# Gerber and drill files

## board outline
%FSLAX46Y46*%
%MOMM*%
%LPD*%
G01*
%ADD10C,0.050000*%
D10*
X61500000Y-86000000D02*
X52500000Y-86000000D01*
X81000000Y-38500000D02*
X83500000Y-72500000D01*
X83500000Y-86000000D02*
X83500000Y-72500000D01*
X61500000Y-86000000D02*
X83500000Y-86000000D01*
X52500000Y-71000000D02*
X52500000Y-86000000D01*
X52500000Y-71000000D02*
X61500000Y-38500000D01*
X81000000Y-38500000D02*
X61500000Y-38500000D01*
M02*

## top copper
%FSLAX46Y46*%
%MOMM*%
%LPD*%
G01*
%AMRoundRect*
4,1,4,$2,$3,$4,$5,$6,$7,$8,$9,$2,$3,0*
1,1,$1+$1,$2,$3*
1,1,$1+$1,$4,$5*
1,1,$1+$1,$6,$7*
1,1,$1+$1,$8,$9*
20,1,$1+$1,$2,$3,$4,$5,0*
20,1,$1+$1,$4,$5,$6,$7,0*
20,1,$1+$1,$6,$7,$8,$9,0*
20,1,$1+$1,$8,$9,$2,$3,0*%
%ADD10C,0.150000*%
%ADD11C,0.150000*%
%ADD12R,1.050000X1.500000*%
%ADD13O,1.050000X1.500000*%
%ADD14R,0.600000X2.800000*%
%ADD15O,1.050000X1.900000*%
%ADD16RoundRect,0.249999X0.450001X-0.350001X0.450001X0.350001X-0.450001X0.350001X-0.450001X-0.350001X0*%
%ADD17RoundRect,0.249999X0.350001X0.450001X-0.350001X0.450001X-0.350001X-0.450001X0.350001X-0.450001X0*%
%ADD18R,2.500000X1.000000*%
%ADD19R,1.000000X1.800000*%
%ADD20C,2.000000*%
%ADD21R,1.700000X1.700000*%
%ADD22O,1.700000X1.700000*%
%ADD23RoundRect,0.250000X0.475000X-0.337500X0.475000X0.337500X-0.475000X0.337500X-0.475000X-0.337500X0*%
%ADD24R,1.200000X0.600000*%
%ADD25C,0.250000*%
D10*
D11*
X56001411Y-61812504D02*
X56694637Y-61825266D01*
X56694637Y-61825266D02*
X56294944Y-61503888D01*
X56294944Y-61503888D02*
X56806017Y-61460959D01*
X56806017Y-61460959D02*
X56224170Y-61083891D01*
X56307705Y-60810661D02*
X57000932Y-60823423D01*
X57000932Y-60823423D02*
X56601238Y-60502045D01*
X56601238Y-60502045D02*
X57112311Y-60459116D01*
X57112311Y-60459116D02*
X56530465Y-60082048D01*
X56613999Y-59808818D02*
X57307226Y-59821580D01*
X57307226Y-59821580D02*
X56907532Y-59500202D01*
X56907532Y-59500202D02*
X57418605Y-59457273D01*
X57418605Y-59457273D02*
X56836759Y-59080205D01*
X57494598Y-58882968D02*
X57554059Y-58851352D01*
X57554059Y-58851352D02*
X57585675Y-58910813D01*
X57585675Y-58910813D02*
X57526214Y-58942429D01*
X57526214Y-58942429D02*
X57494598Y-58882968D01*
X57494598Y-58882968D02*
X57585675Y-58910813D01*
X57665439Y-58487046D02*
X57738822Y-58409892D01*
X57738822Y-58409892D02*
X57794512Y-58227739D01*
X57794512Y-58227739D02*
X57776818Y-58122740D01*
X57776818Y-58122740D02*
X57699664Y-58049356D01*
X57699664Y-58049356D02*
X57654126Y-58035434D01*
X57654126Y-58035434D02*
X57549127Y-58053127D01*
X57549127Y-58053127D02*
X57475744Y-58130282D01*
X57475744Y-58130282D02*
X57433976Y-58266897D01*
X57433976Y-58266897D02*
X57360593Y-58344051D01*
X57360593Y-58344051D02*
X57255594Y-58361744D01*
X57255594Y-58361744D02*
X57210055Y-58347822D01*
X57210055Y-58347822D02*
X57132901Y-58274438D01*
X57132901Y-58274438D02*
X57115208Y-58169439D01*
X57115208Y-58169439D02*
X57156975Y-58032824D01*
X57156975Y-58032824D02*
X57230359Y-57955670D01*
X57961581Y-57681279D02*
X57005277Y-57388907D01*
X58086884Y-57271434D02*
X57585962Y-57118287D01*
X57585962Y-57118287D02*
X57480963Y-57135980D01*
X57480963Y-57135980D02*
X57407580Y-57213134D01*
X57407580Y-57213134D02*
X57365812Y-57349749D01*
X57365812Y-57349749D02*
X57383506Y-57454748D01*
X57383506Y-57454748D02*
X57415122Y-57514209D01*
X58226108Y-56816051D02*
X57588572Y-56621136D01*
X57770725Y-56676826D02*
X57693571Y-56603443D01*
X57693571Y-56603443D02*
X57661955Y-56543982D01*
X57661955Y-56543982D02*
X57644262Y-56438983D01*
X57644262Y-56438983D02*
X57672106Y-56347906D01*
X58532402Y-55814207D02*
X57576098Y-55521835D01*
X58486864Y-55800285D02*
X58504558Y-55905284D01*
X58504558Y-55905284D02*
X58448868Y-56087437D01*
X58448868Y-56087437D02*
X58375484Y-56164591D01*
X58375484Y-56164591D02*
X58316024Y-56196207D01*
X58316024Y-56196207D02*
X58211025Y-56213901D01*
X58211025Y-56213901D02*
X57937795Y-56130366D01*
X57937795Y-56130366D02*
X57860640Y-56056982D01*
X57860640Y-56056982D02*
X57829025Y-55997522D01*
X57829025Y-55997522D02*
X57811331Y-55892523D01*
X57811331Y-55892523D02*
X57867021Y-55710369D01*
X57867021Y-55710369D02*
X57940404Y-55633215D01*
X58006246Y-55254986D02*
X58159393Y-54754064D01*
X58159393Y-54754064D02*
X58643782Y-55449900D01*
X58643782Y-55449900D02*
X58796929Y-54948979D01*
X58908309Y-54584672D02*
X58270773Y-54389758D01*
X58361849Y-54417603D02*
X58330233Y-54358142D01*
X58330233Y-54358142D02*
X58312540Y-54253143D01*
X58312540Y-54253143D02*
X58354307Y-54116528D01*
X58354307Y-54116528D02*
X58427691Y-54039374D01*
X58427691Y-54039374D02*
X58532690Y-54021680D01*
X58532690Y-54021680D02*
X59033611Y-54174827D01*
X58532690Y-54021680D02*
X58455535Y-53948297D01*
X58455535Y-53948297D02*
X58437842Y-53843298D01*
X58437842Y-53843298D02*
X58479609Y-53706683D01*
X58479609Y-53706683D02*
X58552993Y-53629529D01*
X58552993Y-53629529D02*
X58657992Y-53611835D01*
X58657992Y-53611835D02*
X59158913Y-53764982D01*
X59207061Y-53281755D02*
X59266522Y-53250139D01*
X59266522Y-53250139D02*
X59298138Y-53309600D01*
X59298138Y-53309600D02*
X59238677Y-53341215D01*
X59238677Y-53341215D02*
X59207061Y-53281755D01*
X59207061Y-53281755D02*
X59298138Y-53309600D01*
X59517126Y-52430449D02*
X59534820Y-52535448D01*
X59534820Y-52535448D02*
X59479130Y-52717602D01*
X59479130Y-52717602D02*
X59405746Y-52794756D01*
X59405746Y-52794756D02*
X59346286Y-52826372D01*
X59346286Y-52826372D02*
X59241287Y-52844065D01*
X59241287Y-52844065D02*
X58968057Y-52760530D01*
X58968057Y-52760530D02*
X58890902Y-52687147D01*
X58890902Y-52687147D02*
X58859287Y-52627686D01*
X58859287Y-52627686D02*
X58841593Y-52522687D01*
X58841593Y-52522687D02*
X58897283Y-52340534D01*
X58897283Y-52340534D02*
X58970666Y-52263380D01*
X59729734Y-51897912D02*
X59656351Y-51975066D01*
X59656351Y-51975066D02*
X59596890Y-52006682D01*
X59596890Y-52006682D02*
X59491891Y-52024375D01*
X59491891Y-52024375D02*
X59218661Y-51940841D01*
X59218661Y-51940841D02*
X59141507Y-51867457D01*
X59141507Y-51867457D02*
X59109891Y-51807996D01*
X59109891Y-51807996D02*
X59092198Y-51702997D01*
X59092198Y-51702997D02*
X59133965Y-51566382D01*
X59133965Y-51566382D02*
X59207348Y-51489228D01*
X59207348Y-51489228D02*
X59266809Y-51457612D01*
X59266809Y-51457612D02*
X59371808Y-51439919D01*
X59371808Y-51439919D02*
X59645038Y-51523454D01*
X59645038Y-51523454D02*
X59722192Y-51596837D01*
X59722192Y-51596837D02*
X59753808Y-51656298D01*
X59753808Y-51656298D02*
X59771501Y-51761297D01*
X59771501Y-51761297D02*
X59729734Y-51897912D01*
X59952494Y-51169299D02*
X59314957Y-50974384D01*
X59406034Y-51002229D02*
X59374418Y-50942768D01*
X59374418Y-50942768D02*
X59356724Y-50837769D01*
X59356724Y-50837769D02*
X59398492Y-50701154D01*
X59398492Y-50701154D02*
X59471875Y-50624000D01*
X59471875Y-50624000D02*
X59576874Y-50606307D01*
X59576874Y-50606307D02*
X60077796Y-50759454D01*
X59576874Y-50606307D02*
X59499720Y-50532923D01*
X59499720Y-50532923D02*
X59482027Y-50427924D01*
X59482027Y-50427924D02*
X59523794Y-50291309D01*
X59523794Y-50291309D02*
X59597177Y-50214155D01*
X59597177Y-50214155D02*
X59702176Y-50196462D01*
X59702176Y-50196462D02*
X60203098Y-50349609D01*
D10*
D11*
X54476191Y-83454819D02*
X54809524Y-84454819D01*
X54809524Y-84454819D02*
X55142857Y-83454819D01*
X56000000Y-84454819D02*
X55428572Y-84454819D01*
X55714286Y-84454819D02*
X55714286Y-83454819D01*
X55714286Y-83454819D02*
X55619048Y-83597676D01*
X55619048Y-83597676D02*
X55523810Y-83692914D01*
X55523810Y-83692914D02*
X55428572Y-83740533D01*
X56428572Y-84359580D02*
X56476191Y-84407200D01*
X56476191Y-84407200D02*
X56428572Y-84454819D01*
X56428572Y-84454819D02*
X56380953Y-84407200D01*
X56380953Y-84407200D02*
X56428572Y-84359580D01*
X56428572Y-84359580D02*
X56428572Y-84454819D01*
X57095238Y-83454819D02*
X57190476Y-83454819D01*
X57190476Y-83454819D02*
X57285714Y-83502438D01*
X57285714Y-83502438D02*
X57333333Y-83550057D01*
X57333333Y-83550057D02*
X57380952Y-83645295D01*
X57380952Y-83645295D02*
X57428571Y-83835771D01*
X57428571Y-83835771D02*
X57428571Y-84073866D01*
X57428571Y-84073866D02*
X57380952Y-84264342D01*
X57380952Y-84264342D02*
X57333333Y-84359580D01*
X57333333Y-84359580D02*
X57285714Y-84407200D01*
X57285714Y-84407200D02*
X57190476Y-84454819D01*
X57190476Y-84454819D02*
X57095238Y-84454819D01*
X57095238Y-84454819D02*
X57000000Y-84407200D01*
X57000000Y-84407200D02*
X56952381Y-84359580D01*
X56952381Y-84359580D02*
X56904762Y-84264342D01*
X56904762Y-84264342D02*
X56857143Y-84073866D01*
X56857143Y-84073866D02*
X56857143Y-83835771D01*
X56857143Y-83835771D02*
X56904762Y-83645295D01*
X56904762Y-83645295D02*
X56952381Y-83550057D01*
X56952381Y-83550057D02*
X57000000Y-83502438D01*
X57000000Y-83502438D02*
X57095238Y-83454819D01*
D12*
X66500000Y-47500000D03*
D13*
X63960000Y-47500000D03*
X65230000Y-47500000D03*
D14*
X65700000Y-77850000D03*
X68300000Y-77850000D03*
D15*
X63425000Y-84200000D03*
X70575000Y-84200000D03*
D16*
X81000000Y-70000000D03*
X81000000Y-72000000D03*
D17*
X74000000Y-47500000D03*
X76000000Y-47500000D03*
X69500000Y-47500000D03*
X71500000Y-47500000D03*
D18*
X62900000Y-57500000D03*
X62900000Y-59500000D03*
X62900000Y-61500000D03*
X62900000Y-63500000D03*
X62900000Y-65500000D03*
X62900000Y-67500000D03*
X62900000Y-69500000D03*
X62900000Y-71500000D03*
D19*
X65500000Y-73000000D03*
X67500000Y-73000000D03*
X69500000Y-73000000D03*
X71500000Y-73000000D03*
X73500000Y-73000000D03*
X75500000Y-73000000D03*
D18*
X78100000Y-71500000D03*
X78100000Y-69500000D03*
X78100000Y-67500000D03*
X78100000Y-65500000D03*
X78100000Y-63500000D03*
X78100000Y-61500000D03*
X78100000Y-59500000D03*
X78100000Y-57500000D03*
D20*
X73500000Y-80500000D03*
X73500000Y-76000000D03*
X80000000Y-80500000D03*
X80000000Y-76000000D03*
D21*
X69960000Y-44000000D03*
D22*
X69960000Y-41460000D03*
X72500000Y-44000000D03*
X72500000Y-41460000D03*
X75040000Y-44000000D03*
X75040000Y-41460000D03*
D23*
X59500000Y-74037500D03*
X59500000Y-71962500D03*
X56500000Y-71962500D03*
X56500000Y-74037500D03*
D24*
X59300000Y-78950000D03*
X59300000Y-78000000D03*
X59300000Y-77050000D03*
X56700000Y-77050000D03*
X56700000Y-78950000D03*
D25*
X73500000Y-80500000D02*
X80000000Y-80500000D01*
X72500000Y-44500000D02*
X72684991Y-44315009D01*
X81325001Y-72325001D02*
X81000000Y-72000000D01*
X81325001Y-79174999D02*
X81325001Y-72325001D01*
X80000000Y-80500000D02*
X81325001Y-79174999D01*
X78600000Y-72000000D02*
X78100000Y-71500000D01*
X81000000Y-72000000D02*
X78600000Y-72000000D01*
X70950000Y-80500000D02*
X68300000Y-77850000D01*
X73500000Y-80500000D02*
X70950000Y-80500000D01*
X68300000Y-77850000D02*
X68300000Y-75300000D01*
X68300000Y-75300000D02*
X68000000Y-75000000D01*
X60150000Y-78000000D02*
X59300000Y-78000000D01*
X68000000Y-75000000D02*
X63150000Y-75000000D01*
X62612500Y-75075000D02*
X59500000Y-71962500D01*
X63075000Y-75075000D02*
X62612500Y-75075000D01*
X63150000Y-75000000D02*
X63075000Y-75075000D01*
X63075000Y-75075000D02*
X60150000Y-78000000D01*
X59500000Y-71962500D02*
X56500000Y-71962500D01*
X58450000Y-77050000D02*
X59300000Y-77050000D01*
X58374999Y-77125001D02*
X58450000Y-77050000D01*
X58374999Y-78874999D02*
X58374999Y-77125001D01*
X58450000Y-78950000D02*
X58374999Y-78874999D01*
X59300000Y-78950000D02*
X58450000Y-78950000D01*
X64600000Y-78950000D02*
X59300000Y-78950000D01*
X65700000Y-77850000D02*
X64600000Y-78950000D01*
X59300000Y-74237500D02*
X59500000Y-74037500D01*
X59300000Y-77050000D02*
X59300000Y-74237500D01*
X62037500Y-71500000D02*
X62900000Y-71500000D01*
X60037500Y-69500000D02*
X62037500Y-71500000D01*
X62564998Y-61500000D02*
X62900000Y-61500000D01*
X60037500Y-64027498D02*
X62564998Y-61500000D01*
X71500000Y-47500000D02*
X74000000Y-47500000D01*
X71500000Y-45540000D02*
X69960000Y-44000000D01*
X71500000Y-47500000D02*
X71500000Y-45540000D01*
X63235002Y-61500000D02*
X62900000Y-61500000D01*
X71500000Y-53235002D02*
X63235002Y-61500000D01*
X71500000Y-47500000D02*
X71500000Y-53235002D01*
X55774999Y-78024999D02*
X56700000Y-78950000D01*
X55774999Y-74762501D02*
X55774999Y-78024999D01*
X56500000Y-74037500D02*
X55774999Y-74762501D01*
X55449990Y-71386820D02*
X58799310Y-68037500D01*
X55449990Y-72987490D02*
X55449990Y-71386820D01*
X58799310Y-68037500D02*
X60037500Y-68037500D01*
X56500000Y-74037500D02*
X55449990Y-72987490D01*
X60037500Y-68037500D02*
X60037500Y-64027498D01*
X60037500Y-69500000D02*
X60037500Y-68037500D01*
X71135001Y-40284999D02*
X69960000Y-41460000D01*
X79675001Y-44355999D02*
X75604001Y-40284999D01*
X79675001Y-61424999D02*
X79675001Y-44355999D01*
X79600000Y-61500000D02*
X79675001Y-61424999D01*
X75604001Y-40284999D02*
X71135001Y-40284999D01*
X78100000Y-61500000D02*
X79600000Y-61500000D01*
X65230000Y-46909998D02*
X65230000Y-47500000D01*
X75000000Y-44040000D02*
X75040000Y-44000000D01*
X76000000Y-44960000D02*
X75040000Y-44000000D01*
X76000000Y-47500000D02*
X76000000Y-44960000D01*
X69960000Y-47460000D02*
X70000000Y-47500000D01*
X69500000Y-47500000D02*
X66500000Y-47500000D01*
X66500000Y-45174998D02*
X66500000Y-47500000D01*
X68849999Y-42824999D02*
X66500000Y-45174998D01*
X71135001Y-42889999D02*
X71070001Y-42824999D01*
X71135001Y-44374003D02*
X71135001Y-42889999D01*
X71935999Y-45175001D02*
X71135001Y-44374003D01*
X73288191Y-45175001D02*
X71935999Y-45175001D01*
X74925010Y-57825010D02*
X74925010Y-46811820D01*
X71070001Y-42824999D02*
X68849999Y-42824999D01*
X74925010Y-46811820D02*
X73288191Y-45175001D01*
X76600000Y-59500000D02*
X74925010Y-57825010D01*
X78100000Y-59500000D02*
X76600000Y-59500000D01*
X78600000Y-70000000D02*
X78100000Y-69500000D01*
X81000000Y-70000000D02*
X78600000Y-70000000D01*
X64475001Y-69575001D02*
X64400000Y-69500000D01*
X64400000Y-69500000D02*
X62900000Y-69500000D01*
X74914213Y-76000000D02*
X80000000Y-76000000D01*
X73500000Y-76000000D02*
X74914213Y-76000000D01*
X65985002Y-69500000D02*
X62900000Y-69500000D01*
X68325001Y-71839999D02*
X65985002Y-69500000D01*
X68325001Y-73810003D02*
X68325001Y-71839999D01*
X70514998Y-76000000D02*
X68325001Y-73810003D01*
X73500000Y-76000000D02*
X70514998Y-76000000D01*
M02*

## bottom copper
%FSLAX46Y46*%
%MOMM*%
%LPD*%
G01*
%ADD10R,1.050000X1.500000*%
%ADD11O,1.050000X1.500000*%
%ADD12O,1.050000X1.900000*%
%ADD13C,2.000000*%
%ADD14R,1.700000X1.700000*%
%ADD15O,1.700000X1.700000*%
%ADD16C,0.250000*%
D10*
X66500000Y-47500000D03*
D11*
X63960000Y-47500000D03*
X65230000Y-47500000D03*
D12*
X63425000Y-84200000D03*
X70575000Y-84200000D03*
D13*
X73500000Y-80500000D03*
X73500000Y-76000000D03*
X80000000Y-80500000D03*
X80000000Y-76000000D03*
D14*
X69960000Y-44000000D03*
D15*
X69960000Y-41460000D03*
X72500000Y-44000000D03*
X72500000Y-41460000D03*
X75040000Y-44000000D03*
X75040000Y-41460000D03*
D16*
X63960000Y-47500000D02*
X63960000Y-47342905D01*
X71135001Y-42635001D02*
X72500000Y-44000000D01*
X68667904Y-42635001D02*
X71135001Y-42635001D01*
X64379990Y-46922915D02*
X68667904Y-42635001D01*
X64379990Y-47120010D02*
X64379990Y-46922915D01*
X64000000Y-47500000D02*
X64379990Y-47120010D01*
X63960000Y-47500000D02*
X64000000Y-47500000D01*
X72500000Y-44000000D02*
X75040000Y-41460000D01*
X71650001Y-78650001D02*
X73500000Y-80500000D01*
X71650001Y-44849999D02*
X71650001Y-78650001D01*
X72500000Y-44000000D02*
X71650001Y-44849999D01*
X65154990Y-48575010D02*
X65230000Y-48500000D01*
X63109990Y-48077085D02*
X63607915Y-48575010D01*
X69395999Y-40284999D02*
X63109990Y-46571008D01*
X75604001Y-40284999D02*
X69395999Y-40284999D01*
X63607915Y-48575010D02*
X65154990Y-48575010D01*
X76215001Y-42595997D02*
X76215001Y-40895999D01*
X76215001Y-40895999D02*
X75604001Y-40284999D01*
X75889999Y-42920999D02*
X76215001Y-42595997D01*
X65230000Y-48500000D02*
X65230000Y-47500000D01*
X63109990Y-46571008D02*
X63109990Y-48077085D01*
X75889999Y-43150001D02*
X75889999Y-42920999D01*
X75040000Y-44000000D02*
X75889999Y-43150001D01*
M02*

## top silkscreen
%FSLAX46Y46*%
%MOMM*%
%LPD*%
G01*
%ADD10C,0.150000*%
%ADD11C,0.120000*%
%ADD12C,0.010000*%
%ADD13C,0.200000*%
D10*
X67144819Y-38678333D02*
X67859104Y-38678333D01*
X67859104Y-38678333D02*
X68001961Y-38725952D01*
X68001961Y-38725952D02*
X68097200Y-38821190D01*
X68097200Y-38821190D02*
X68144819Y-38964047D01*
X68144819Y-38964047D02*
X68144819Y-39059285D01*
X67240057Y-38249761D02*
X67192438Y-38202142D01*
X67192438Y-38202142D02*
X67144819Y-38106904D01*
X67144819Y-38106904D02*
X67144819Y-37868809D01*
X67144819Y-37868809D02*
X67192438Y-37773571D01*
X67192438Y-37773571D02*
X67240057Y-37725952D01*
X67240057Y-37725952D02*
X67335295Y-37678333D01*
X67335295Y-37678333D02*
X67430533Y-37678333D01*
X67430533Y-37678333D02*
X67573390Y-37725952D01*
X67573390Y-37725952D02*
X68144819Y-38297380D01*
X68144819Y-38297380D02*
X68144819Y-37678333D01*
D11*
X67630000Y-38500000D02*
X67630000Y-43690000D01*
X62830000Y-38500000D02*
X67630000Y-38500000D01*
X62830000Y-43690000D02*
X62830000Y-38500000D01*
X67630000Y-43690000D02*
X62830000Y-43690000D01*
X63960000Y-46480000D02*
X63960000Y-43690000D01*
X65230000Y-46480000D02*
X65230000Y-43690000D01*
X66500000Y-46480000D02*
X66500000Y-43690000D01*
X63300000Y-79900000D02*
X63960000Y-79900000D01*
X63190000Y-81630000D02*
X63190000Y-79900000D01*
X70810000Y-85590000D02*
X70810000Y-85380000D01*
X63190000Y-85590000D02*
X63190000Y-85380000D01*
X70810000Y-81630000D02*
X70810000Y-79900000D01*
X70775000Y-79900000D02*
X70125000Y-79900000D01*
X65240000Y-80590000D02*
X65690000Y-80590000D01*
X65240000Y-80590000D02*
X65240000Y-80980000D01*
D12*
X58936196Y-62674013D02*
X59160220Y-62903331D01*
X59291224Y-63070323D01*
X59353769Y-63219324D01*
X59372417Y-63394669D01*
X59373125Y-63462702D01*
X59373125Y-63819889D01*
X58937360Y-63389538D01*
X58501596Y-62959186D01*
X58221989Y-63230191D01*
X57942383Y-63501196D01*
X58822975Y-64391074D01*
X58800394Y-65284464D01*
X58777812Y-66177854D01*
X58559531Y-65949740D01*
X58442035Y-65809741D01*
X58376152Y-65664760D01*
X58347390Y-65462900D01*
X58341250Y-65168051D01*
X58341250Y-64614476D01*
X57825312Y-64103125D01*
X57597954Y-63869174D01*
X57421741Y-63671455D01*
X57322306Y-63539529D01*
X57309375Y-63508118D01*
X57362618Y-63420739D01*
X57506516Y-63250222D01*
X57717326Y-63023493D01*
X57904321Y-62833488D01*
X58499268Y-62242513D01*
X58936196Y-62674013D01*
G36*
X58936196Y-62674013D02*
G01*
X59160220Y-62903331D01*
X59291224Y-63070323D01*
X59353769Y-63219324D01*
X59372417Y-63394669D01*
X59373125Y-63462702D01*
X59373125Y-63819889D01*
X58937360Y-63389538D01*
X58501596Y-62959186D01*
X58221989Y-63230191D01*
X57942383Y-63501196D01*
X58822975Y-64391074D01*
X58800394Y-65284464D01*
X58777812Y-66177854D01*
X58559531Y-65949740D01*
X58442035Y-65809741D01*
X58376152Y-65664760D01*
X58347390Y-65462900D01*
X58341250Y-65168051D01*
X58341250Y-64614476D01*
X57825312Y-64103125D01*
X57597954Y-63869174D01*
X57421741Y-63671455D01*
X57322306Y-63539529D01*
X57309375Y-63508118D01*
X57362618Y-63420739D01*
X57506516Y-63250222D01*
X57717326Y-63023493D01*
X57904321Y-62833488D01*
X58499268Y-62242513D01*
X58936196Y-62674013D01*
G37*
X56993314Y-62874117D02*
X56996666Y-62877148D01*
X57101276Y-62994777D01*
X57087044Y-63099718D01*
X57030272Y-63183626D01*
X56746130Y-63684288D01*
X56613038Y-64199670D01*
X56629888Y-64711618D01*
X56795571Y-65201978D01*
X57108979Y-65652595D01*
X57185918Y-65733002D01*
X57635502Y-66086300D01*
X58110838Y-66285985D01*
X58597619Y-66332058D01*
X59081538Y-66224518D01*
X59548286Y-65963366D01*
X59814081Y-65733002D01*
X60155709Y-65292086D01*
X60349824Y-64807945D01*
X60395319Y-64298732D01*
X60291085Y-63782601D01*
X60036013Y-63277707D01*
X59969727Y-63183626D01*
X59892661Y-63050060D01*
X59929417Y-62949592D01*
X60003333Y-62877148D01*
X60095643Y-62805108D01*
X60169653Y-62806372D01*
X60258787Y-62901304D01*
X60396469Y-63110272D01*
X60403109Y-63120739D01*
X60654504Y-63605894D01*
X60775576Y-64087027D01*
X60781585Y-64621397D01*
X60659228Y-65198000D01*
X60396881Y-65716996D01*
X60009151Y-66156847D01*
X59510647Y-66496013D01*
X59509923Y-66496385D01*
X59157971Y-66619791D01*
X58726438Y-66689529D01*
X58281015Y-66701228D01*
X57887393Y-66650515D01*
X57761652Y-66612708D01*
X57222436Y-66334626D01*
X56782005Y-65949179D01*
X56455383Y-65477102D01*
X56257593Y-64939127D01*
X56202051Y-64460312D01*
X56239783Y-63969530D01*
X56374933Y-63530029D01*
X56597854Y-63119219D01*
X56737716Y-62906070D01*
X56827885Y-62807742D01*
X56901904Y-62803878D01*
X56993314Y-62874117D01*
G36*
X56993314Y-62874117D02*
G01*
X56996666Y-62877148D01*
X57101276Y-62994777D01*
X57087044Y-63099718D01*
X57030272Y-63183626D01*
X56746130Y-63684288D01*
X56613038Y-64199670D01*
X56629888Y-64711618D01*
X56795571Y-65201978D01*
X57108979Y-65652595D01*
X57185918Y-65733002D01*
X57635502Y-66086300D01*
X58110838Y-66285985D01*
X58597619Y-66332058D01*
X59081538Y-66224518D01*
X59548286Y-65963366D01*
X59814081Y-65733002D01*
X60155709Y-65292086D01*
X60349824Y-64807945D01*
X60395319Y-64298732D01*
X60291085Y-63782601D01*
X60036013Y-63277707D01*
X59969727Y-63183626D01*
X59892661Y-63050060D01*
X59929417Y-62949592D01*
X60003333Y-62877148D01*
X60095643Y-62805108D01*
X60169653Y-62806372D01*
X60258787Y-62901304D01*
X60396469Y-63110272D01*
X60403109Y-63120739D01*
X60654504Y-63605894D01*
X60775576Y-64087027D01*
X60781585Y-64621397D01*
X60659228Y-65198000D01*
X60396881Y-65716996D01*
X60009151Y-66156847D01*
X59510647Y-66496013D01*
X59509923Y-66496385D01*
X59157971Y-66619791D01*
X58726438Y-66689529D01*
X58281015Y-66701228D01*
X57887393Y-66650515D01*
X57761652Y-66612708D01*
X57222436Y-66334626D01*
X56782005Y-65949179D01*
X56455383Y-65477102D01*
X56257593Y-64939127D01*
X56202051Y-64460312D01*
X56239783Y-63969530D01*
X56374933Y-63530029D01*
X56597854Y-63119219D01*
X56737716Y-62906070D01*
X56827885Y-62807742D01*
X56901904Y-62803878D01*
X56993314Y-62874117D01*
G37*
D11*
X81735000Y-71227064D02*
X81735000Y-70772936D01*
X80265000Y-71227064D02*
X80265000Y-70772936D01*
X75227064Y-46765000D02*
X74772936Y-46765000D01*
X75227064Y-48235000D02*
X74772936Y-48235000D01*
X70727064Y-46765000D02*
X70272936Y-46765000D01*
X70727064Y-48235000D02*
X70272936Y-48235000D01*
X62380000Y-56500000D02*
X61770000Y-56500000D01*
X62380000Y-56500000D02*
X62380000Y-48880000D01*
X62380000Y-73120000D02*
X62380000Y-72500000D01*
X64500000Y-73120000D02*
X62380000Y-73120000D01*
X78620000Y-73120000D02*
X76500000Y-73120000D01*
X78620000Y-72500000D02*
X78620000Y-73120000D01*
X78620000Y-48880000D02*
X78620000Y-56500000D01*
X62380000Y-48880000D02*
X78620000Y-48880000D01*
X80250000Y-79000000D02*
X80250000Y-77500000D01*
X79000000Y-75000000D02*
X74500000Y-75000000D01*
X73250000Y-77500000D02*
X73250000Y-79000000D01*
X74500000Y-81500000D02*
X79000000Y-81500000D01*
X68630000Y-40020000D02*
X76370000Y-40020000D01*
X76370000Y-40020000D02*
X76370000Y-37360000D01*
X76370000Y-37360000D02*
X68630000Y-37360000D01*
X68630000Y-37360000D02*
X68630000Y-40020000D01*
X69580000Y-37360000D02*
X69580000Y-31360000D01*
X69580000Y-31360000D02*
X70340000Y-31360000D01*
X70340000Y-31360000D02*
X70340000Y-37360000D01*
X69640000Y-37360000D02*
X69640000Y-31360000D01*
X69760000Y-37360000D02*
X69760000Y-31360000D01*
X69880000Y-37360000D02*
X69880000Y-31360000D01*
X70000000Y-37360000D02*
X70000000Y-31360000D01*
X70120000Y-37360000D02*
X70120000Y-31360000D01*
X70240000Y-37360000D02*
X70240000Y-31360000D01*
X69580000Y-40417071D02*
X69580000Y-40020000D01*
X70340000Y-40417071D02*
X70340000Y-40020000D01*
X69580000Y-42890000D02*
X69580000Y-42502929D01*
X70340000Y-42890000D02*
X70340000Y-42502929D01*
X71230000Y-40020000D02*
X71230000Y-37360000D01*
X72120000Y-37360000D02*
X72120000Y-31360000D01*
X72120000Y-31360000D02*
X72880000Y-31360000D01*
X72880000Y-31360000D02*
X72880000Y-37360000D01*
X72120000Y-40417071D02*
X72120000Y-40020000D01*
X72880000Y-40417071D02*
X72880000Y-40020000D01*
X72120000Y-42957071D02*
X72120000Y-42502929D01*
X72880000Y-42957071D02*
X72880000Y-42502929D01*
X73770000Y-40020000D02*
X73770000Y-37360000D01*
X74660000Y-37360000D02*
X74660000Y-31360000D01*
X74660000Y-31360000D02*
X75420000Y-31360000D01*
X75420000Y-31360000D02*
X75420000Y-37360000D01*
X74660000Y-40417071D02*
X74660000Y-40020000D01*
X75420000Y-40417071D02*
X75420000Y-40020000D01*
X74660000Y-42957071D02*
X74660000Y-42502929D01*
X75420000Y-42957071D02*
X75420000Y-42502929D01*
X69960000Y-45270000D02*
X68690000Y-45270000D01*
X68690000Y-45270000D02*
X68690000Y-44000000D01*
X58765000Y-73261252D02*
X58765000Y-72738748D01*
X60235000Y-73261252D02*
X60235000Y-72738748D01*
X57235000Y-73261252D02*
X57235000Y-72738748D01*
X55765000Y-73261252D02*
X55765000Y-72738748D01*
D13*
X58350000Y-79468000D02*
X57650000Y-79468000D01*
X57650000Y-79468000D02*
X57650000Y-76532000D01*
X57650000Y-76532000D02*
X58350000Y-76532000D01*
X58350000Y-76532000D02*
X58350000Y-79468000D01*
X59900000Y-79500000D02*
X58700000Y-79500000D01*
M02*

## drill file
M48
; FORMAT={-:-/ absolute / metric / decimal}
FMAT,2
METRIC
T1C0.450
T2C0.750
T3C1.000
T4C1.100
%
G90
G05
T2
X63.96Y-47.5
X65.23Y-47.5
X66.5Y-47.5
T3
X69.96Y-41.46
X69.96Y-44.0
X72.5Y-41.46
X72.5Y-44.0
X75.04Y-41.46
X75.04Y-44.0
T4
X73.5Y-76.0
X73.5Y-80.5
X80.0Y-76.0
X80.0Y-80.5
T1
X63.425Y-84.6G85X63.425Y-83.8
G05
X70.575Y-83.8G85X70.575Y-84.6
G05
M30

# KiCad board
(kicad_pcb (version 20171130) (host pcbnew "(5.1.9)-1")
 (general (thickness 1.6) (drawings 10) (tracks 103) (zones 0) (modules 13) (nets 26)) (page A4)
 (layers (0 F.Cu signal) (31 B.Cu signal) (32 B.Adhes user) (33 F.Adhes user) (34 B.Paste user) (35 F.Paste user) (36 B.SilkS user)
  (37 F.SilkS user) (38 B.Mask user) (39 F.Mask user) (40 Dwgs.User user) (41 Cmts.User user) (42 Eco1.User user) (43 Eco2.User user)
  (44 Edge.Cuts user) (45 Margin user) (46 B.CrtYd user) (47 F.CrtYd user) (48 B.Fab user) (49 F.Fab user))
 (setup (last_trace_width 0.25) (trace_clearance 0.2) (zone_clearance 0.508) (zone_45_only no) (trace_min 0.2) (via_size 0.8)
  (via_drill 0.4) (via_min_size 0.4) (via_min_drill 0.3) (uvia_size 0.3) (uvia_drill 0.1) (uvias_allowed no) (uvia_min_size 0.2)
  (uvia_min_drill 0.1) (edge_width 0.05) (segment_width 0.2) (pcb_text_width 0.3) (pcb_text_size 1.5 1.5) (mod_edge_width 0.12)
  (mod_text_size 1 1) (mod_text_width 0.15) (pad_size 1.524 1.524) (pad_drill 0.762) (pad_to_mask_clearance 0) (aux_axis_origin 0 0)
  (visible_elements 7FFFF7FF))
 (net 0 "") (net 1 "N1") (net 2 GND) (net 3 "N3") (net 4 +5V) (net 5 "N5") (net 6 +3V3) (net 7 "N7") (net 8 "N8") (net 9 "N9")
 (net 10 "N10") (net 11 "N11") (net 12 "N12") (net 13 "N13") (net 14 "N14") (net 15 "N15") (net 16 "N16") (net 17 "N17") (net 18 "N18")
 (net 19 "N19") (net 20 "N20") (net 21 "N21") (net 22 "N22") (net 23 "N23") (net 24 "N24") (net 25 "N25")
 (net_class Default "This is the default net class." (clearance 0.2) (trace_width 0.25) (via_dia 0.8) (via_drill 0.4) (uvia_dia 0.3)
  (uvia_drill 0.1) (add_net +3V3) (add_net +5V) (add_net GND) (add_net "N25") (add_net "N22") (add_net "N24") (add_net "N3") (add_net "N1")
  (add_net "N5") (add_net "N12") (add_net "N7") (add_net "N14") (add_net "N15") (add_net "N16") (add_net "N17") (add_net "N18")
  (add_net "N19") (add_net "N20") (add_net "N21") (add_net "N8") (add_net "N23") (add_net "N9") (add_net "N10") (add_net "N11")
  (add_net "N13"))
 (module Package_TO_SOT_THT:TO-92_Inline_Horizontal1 (layer F.Cu) (at 66.5 47.5 180)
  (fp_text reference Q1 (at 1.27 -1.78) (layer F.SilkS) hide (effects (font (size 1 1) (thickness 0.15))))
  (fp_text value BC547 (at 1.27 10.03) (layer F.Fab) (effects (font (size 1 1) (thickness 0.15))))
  (fp_line (start -1.13 9) (end -1.13 3.81) (layer F.SilkS) (width 0.12))
  (fp_line (start 3.67 9) (end -1.13 9) (layer F.SilkS) (width 0.12))
  (fp_line (start 3.67 3.81) (end 3.67 9) (layer F.SilkS) (width 0.12))
  (fp_line (start -1.13 3.81) (end 3.67 3.81) (layer F.SilkS) (width 0.12))
  (fp_line (start 2.54 1.02) (end 2.54 3.81) (layer F.SilkS) (width 0.12))
  (fp_line (start 1.27 1.02) (end 1.27 3.81) (layer F.SilkS) (width 0.12))
  (fp_line (start 0 1.02) (end 0 3.81) (layer F.SilkS) (width 0.12))
  (pad 1 thru_hole rect (at 0 0 180) (size 1.05 1.5) (drill 0.75) (layers *.Cu *.Mask) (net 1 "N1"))
  (pad 3 thru_hole oval (at 2.54 0 180) (size 1.05 1.5) (drill 0.75) (layers *.Cu *.Mask) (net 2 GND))
  (pad 2 thru_hole oval (at 1.27 0 180) (size 1.05 1.5) (drill 0.75) (layers *.Cu *.Mask) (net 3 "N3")))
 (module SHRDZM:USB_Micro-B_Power (layer F.Cu) (at 67 83)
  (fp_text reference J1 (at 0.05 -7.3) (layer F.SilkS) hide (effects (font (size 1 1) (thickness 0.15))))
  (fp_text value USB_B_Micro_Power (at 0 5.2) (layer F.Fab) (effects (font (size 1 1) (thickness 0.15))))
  (fp_line (start -3.7 -3.1) (end -3.04 -3.1) (layer F.SilkS) (width 0.12))
  (fp_line (start -3.81 -1.37) (end -3.81 -3.1) (layer F.SilkS) (width 0.12))
  (fp_line (start 3.81 2.59) (end 3.81 2.38) (layer F.SilkS) (width 0.12))
  (fp_line (start -3.81 2.59) (end -3.81 2.38) (layer F.SilkS) (width 0.12))
  (fp_line (start 3.81 -1.37) (end 3.81 -3.1) (layer F.SilkS) (width 0.12))
  (fp_line (start 3.775 -3.1) (end 3.125 -3.1) (layer F.SilkS) (width 0.12))
  (fp_line (start -1.76 -2.41) (end -1.31 -2.41) (layer F.SilkS) (width 0.12))
  (fp_line (start -1.76 -2.41) (end -1.76 -2.02) (layer F.SilkS) (width 0.12))
  (pad 1 smd rect (at -1.3 -5.15) (size 0.6 2.8) (layers F.Cu F.Paste F.Mask) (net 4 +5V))
  (pad 5 smd rect (at 1.3 -5.15) (size 0.6 2.8) (layers F.Cu F.Paste F.Mask) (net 2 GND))
  (pad "" thru_hole oval (at -3.575 1.2 180) (size 1.05 1.9) (drill oval 0.45 1.25) (layers *.Cu *.Mask))
  (pad "" thru_hole oval (at 3.575 1.2) (size 1.05 1.9) (drill oval 0.45 1.25) (layers *.Cu *.Mask)))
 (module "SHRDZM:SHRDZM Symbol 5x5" (layer F.Cu) (at 58.5 64.5)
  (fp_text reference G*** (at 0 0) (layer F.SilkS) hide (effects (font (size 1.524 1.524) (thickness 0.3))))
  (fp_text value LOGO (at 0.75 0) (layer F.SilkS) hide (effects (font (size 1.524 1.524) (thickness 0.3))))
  (fp_poly
   (pts (xy 0.436196 -1.825987) (xy 0.66022 -1.596669) (xy 0.791224 -1.429677) (xy 0.853769 -1.280676) (xy 0.872417 -1.105331)
    (xy 0.873125 -1.037298) (xy 0.873125 -0.680111) (xy 0.43736 -1.110462) (xy 0.001596 -1.540814) (xy -0.278011 -1.269809)
    (xy -0.557617 -0.998804) (xy 0.322975 -0.108926) (xy 0.300394 0.784464) (xy 0.277812 1.677854) (xy 0.059531 1.44974)
    (xy -0.057965 1.309741) (xy -0.123848 1.16476) (xy -0.15261 0.9629) (xy -0.15875 0.668051) (xy -0.15875 0.114476)
    (xy -0.674688 -0.396875) (xy -0.902046 -0.630826) (xy -1.078259 -0.828545) (xy -1.177694 -0.960471) (xy -1.190625 -0.991882)
    (xy -1.137382 -1.079261) (xy -0.993484 -1.249778) (xy -0.782674 -1.476507) (xy -0.595679 -1.666512) (xy -0.000732 -2.257487)
    (xy 0.436196 -1.825987))
   (layer F.SilkS) (width 0.01))
  (fp_poly
   (pts (xy -1.506686 -1.625883) (xy -1.503334 -1.622852) (xy -1.398724 -1.505223) (xy -1.412956 -1.400282) (xy -1.469728 -1.316374)
    (xy -1.75387 -0.815712) (xy -1.886962 -0.30033) (xy -1.870112 0.211618) (xy -1.704429 0.701978) (xy -1.391021 1.152595)
    (xy -1.314082 1.233002) (xy -0.864498 1.5863) (xy -0.389162 1.785985) (xy 0.097619 1.832058) (xy 0.581538 1.724518)
    (xy 1.048286 1.463366) (xy 1.314081 1.233002) (xy 1.655709 0.792086) (xy 1.849824 0.307945) (xy 1.895319 -0.201268)
    (xy 1.791085 -0.717399) (xy 1.536013 -1.222293) (xy 1.469727 -1.316374) (xy 1.392661 -1.44994) (xy 1.429417 -1.550408)
    (xy 1.503333 -1.622852) (xy 1.595643 -1.694892) (xy 1.669653 -1.693628) (xy 1.758787 -1.598696) (xy 1.896469 -1.389728)
    (xy 1.903109 -1.379261) (xy 2.154504 -0.894106) (xy 2.275576 -0.412973) (xy 2.281585 0.121397) (xy 2.159228 0.698)
    (xy 1.896881 1.216996) (xy 1.509151 1.656847) (xy 1.010647 1.996013) (xy 1.009923 1.996385) (xy 0.657971 2.119791)
    (xy 0.226438 2.189529) (xy -0.218985 2.201228) (xy -0.612607 2.150515) (xy -0.738348 2.112708) (xy -1.277564 1.834626)
    (xy -1.717995 1.449179) (xy -2.044617 0.977102) (xy -2.242407 0.439127) (xy -2.297949 -0.039688) (xy -2.260217 -0.53047)
    (xy -2.125067 -0.969971) (xy -1.902146 -1.380781) (xy -1.762284 -1.59393) (xy -1.672115 -1.692258) (xy -1.598096 -1.696122)
    (xy -1.506686 -1.625883))
   (layer F.SilkS) (width 0.01)))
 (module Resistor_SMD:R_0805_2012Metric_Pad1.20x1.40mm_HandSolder (layer F.Cu) (at 81 71 90)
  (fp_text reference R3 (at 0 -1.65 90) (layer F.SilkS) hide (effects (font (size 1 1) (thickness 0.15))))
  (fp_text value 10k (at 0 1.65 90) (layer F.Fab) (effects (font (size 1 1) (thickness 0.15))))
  (fp_line (start -0.227064 0.735) (end 0.227064 0.735) (layer F.SilkS) (width 0.12))
  (fp_line (start -0.227064 -0.735) (end 0.227064 -0.735) (layer F.SilkS) (width 0.12))
  (pad 2 smd roundrect (at 1 0 90) (size 1.2 1.4) (layers F.Cu F.Paste F.Mask) (roundrect_rratio 0.2083325) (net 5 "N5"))
  (pad 1 smd roundrect (at -1 0 90) (size 1.2 1.4) (layers F.Cu F.Paste F.Mask) (roundrect_rratio 0.2083325) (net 2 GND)))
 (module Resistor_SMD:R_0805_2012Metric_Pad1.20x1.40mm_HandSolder (layer F.Cu) (at 75 47.5 180)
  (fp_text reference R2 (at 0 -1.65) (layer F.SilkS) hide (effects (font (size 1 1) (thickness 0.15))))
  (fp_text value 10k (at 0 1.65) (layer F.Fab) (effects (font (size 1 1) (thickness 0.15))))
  (fp_line (start -0.227064 0.735) (end 0.227064 0.735) (layer F.SilkS) (width 0.12))
  (fp_line (start -0.227064 -0.735) (end 0.227064 -0.735) (layer F.SilkS) (width 0.12))
  (pad 2 smd roundrect (at 1 0 180) (size 1.2 1.4) (layers F.Cu F.Paste F.Mask) (roundrect_rratio 0.2083325) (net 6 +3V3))
  (pad 1 smd roundrect (at -1 0 180) (size 1.2 1.4) (layers F.Cu F.Paste F.Mask) (roundrect_rratio 0.2083325) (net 3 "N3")))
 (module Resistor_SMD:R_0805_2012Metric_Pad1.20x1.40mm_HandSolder (layer F.Cu) (at 70.5 47.5 180)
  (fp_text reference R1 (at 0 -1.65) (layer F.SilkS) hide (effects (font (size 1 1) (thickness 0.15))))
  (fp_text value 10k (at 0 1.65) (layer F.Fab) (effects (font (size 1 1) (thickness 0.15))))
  (fp_line (start -0.227064 0.735) (end 0.227064 0.735) (layer F.SilkS) (width 0.12))
  (fp_line (start -0.227064 -0.735) (end 0.227064 -0.735) (layer F.SilkS) (width 0.12))
  (pad 2 smd roundrect (at 1 0 180) (size 1.2 1.4) (layers F.Cu F.Paste F.Mask) (roundrect_rratio 0.2083325) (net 1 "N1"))
  (pad 1 smd roundrect (at -1 0 180) (size 1.2 1.4) (layers F.Cu F.Paste F.Mask) (roundrect_rratio 0.2083325) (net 6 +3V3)))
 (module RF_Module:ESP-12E (layer F.Cu) (at 70.5 61)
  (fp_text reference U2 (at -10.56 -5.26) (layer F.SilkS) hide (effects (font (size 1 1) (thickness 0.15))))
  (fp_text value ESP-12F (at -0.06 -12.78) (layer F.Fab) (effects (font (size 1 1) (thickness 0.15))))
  (fp_line (start -8.12 -4.5) (end -8.73 -4.5) (layer F.SilkS) (width 0.12))
  (fp_line (start -8.12 -4.5) (end -8.12 -12.12) (layer F.SilkS) (width 0.12))
  (fp_line (start -8.12 12.12) (end -8.12 11.5) (layer F.SilkS) (width 0.12))
  (fp_line (start -6 12.12) (end -8.12 12.12) (layer F.SilkS) (width 0.12))
  (fp_line (start 8.12 12.12) (end 6 12.12) (layer F.SilkS) (width 0.12))
  (fp_line (start 8.12 11.5) (end 8.12 12.12) (layer F.SilkS) (width 0.12))
  (fp_line (start 8.12 -12.12) (end 8.12 -4.5) (layer F.SilkS) (width 0.12))
  (fp_line (start -8.12 -12.12) (end 8.12 -12.12) (layer F.SilkS) (width 0.12))
  (pad 1 smd rect (at -7.6 -3.5) (size 2.5 1) (layers F.Cu F.Paste F.Mask) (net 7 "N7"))
  (pad 2 smd rect (at -7.6 -1.5) (size 2.5 1) (layers F.Cu F.Paste F.Mask) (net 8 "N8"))
  (pad 3 smd rect (at -7.6 0.5) (size 2.5 1) (layers F.Cu F.Paste F.Mask) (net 6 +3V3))
  (pad 4 smd rect (at -7.6 2.5) (size 2.5 1) (layers F.Cu F.Paste F.Mask) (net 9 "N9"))
  (pad 5 smd rect (at -7.6 4.5) (size 2.5 1) (layers F.Cu F.Paste F.Mask) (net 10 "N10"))
  (pad 6 smd rect (at -7.6 6.5) (size 2.5 1) (layers F.Cu F.Paste F.Mask) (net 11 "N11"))
  (pad 7 smd rect (at -7.6 8.5) (size 2.5 1) (layers F.Cu F.Paste F.Mask) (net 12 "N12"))
  (pad 8 smd rect (at -7.6 10.5) (size 2.5 1) (layers F.Cu F.Paste F.Mask) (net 6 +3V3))
  (pad 9 smd rect (at -5 12) (size 1 1.8) (layers F.Cu F.Paste F.Mask) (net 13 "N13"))
  (pad 10 smd rect (at -3 12) (size 1 1.8) (layers F.Cu F.Paste F.Mask) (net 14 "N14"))
  (pad 11 smd rect (at -1 12) (size 1 1.8) (layers F.Cu F.Paste F.Mask) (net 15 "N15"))
  (pad 12 smd rect (at 1 12) (size 1 1.8) (layers F.Cu F.Paste F.Mask) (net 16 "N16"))
  (pad 13 smd rect (at 3 12) (size 1 1.8) (layers F.Cu F.Paste F.Mask) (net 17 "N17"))
  (pad 14 smd rect (at 5 12) (size 1 1.8) (layers F.Cu F.Paste F.Mask) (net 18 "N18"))
  (pad 15 smd rect (at 7.6 10.5) (size 2.5 1) (layers F.Cu F.Paste F.Mask) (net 2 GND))
  (pad 16 smd rect (at 7.6 8.5) (size 2.5 1) (layers F.Cu F.Paste F.Mask) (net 5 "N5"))
  (pad 17 smd rect (at 7.6 6.5) (size 2.5 1) (layers F.Cu F.Paste F.Mask) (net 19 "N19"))
  (pad 18 smd rect (at 7.6 4.5) (size 2.5 1) (layers F.Cu F.Paste F.Mask) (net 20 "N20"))
  (pad 19 smd rect (at 7.6 2.5) (size 2.5 1) (layers F.Cu F.Paste F.Mask) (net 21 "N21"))
  (pad 20 smd rect (at 7.6 0.5) (size 2.5 1) (layers F.Cu F.Paste F.Mask) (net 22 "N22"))
  (pad 21 smd rect (at 7.6 -1.5) (size 2.5 1) (layers F.Cu F.Paste F.Mask) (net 1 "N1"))
  (pad 22 smd rect (at 7.6 -3.5) (size 2.5 1) (layers F.Cu F.Paste F.Mask) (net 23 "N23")))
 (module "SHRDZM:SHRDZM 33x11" (layer B.Cu) (at 66 65 270)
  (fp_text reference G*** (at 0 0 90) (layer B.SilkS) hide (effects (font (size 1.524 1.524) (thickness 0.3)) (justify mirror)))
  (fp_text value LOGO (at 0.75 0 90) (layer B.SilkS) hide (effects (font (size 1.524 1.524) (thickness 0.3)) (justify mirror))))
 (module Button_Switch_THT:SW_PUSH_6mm (layer F.Cu) (at 73.5 76)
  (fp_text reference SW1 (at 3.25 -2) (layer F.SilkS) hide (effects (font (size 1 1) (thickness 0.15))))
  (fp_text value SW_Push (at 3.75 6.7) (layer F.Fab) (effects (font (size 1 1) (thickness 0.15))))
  (fp_line (start 6.75 3) (end 6.75 1.5) (layer F.SilkS) (width 0.12))
  (fp_line (start 5.5 -1) (end 1 -1) (layer F.SilkS) (width 0.12))
  (fp_line (start -0.25 1.5) (end -0.25 3) (layer F.SilkS) (width 0.12))
  (fp_line (start 1 5.5) (end 5.5 5.5) (layer F.SilkS) (width 0.12))
  (pad 2 thru_hole circle (at 0 4.5 90) (size 2 2) (drill 1.1) (layers *.Cu *.Mask) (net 2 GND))
  (pad 1 thru_hole circle (at 0 0 90) (size 2 2) (drill 1.1) (layers *.Cu *.Mask) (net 12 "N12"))
  (pad 2 thru_hole circle (at 6.5 4.5 90) (size 2 2) (drill 1.1) (layers *.Cu *.Mask) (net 2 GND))
  (pad 1 thru_hole circle (at 6.5 0 90) (size 2 2) (drill 1.1) (layers *.Cu *.Mask) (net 12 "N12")))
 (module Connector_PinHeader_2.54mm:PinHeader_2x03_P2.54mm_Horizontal (layer F.Cu) (at 69.96 44 90)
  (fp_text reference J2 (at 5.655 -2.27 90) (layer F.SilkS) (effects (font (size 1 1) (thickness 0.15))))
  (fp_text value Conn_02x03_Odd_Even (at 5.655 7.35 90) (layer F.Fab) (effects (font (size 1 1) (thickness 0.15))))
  (fp_line (start 3.98 -1.33) (end 3.98 6.41) (layer F.SilkS) (width 0.12))
  (fp_line (start 3.98 6.41) (end 6.64 6.41) (layer F.SilkS) (width 0.12))
  (fp_line (start 6.64 6.41) (end 6.64 -1.33) (layer F.SilkS) (width 0.12))
  (fp_line (start 6.64 -1.33) (end 3.98 -1.33) (layer F.SilkS) (width 0.12))
  (fp_line (start 6.64 -0.38) (end 12.64 -0.38) (layer F.SilkS) (width 0.12))
  (fp_line (start 12.64 -0.38) (end 12.64 0.38) (layer F.SilkS) (width 0.12))
  (fp_line (start 12.64 0.38) (end 6.64 0.38) (layer F.SilkS) (width 0.12))
  (fp_line (start 6.64 -0.32) (end 12.64 -0.32) (layer F.SilkS) (width 0.12))
  (fp_line (start 6.64 -0.2) (end 12.64 -0.2) (layer F.SilkS) (width 0.12))
  (fp_line (start 6.64 -0.08) (end 12.64 -0.08) (layer F.SilkS) (width 0.12))
  (fp_line (start 6.64 0.04) (end 12.64 0.04) (layer F.SilkS) (width 0.12))
  (fp_line (start 6.64 0.16) (end 12.64 0.16) (layer F.SilkS) (width 0.12))
  (fp_line (start 6.64 0.28) (end 12.64 0.28) (layer F.SilkS) (width 0.12))
  (fp_line (start 3.582929 -0.38) (end 3.98 -0.38) (layer F.SilkS) (width 0.12))
  (fp_line (start 3.582929 0.38) (end 3.98 0.38) (layer F.SilkS) (width 0.12))
  (fp_line (start 1.11 -0.38) (end 1.497071 -0.38) (layer F.SilkS) (width 0.12))
  (fp_line (start 1.11 0.38) (end 1.497071 0.38) (layer F.SilkS) (width 0.12))
  (fp_line (start 3.98 1.27) (end 6.64 1.27) (layer F.SilkS) (width 0.12))
  (fp_line (start 6.64 2.16) (end 12.64 2.16) (layer F.SilkS) (width 0.12))
  (fp_line (start 12.64 2.16) (end 12.64 2.92) (layer F.SilkS) (width 0.12))
  (fp_line (start 12.64 2.92) (end 6.64 2.92) (layer F.SilkS) (width 0.12))
  (fp_line (start 3.582929 2.16) (end 3.98 2.16) (layer F.SilkS) (width 0.12))
  (fp_line (start 3.582929 2.92) (end 3.98 2.92) (layer F.SilkS) (width 0.12))
  (fp_line (start 1.042929 2.16) (end 1.497071 2.16) (layer F.SilkS) (width 0.12))
  (fp_line (start 1.042929 2.92) (end 1.497071 2.92) (layer F.SilkS) (width 0.12))
  (fp_line (start 3.98 3.81) (end 6.64 3.81) (layer F.SilkS) (width 0.12))
  (fp_line (start 6.64 4.7) (end 12.64 4.7) (layer F.SilkS) (width 0.12))
  (fp_line (start 12.64 4.7) (end 12.64 5.46) (layer F.SilkS) (width 0.12))
  (fp_line (start 12.64 5.46) (end 6.64 5.46) (layer F.SilkS) (width 0.12))
  (fp_line (start 3.582929 4.7) (end 3.98 4.7) (layer F.SilkS) (width 0.12))
  (fp_line (start 3.582929 5.46) (end 3.98 5.46) (layer F.SilkS) (width 0.12))
  (fp_line (start 1.042929 4.7) (end 1.497071 4.7) (layer F.SilkS) (width 0.12))
  (fp_line (start 1.042929 5.46) (end 1.497071 5.46) (layer F.SilkS) (width 0.12))
  (fp_line (start -1.27 0) (end -1.27 -1.27) (layer F.SilkS) (width 0.12))
  (fp_line (start -1.27 -1.27) (end 0 -1.27) (layer F.SilkS) (width 0.12))
  (pad 1 thru_hole rect (at 0 0 90) (size 1.7 1.7) (drill 1) (layers *.Cu *.Mask) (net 6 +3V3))
  (pad 2 thru_hole oval (at 2.54 0 90) (size 1.7 1.7) (drill 1) (layers *.Cu *.Mask) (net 22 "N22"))
  (pad 3 thru_hole oval (at 0 2.54 90) (size 1.7 1.7) (drill 1) (layers *.Cu *.Mask) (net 2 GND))
  (pad 4 thru_hole oval (at 2.54 2.54 90) (size 1.7 1.7) (drill 1) (layers *.Cu *.Mask) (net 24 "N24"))
  (pad 5 thru_hole oval (at 0 5.08 90) (size 1.7 1.7) (drill 1) (layers *.Cu *.Mask) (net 3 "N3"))
  (pad 6 thru_hole oval (at 2.54 5.08 90) (size 1.7 1.7) (drill 1) (layers *.Cu *.Mask) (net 2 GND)))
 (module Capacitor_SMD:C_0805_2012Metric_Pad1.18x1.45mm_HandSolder (layer F.Cu) (at 59.5 73 90)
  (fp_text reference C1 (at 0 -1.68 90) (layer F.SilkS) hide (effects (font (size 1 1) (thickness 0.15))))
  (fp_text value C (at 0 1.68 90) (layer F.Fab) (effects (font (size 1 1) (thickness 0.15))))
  (fp_line (start -0.261252 -0.735) (end 0.261252 -0.735) (layer F.SilkS) (width 0.12))
  (fp_line (start -0.261252 0.735) (end 0.261252 0.735) (layer F.SilkS) (width 0.12))
  (pad 1 smd roundrect (at -1.0375 0 90) (size 1.175 1.45) (layers F.Cu F.Paste F.Mask) (roundrect_rratio 0.212766) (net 4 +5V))
  (pad 2 smd roundrect (at 1.0375 0 90) (size 1.175 1.45) (layers F.Cu F.Paste F.Mask) (roundrect_rratio 0.212766) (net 2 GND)))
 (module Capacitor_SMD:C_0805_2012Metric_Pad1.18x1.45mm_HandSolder (layer F.Cu) (at 56.5 73 90)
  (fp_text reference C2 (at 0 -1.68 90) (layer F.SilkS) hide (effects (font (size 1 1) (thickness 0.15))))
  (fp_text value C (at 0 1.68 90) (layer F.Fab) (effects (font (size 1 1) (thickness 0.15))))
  (fp_line (start -0.261252 0.735) (end 0.261252 0.735) (layer F.SilkS) (width 0.12))
  (fp_line (start -0.261252 -0.735) (end 0.261252 -0.735) (layer F.SilkS) (width 0.12))
  (pad 2 smd roundrect (at 1.0375 0 90) (size 1.175 1.45) (layers F.Cu F.Paste F.Mask) (roundrect_rratio 0.212766) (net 2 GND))
  (pad 1 smd roundrect (at -1.0375 0 90) (size 1.175 1.45) (layers F.Cu F.Paste F.Mask) (roundrect_rratio 0.212766) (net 6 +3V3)))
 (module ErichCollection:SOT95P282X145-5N (layer F.Cu) (at 58 78 180)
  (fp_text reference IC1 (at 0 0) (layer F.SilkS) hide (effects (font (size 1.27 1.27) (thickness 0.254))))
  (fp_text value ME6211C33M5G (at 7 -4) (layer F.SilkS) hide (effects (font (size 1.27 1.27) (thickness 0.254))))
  (fp_line (start -0.35 -1.468) (end 0.35 -1.468) (layer F.SilkS) (width 0.2))
  (fp_line (start 0.35 -1.468) (end 0.35 1.468) (layer F.SilkS) (width 0.2))
  (fp_line (start 0.35 1.468) (end -0.35 1.468) (layer F.SilkS) (width 0.2))
  (fp_line (start -0.35 1.468) (end -0.35 -1.468) (layer F.SilkS) (width 0.2))
  (fp_line (start -1.9 -1.5) (end -0.7 -1.5) (layer F.SilkS) (width 0.2))
  (pad 1 smd rect (at -1.3 -0.95 270) (size 0.6 1.2) (layers F.Cu F.Paste F.Mask) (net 4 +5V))
  (pad 2 smd rect (at -1.3 0 270) (size 0.6 1.2) (layers F.Cu F.Paste F.Mask) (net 2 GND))
  (pad 3 smd rect (at -1.3 0.95 270) (size 0.6 1.2) (layers F.Cu F.Paste F.Mask) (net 4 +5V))
  (pad 4 smd rect (at 1.3 0.95 270) (size 0.6 1.2) (layers F.Cu F.Paste F.Mask) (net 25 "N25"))
  (pad 5 smd rect (at 1.3 -0.95 270) (size 0.6 1.2) (layers F.Cu F.Paste F.Mask) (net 6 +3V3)))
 (gr_line (start 61.5 86) (end 52.5 86) (layer Edge.Cuts) (width 0.05))
 (gr_line (start 81 38.5) (end 83.5 72.5) (layer Edge.Cuts) (width 0.05))
 (gr_line (start 83.5 86) (end 83.5 72.5) (layer Edge.Cuts) (width 0.05))
 (gr_line (start 61.5 86) (end 83.5 86) (layer Edge.Cuts) (width 0.05))
 (gr_line (start 52.5 71) (end 52.5 86) (layer Edge.Cuts) (width 0.05))
 (gr_line (start 52.5 71) (end 61.5 38.5) (layer Edge.Cuts) (width 0.05))
 (gr_line (start 81 38.5) (end 61.5 38.5) (layer Edge.Cuts) (width 0.05))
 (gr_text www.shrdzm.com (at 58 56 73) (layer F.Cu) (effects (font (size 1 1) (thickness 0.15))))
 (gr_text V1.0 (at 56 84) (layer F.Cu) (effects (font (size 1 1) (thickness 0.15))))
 (segment (start 73.5 80.5) (end 80 80.5) (width 0.25) (layer F.Cu) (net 2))
 (segment (start 72.5 44.5) (end 72.684991 44.315009) (width 0.25) (layer F.Cu) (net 2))
 (segment (start 63.96 47.5) (end 63.96 47.342905) (width 0.25) (layer B.Cu) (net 2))
 (segment (start 81.325001 72.325001) (end 81 72) (width 0.25) (layer F.Cu) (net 2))
 (segment (start 81.325001 79.174999) (end 81.325001 72.325001) (width 0.25) (layer F.Cu) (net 2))
 (segment (start 80 80.5) (end 81.325001 79.174999) (width 0.25) (layer F.Cu) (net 2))
 (segment (start 78.6 72) (end 78.1 71.5) (width 0.25) (layer F.Cu) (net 2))
 (segment (start 81 72) (end 78.6 72) (width 0.25) (layer F.Cu) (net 2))
 (segment (start 71.135001 42.635001) (end 72.5 44) (width 0.25) (layer B.Cu) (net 2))
 (segment (start 68.667904 42.635001) (end 71.135001 42.635001) (width 0.25) (layer B.Cu) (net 2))
 (segment (start 64.37999 46.922915) (end 68.667904 42.635001) (width 0.25) (layer B.Cu) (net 2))
 (segment (start 64.37999 47.12001) (end 64.37999 46.922915) (width 0.25) (layer B.Cu) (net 2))
 (segment (start 64 47.5) (end 64.37999 47.12001) (width 0.25) (layer B.Cu) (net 2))
 (segment (start 63.96 47.5) (end 64 47.5) (width 0.25) (layer B.Cu) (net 2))
 (segment (start 72.5 44) (end 75.04 41.46) (width 0.25) (layer B.Cu) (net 2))
 (segment (start 71.650001 78.650001) (end 73.5 80.5) (width 0.25) (layer B.Cu) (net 2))
 (segment (start 71.650001 44.849999) (end 71.650001 78.650001) (width 0.25) (layer B.Cu) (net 2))
 (segment (start 72.5 44) (end 71.650001 44.849999) (width 0.25) (layer B.Cu) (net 2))
 (segment (start 70.95 80.5) (end 68.3 77.85) (width 0.25) (layer F.Cu) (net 2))
 (segment (start 73.5 80.5) (end 70.95 80.5) (width 0.25) (layer F.Cu) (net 2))
 (segment (start 68.3 77.85) (end 68.3 75.3) (width 0.25) (layer F.Cu) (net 2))
 (segment (start 68.3 75.3) (end 68 75) (width 0.25) (layer F.Cu) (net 2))
 (segment (start 60.15 78) (end 59.3 78) (width 0.25) (layer F.Cu) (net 2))
 (segment (start 68 75) (end 63.15 75) (width 0.25) (layer F.Cu) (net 2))
 (segment (start 62.6125 75.075) (end 59.5 71.9625) (width 0.25) (layer F.Cu) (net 2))
 (segment (start 63.075 75.075) (end 62.6125 75.075) (width 0.25) (layer F.Cu) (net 2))
 (segment (start 63.15 75) (end 63.075 75.075) (width 0.25) (layer F.Cu) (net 2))
 (segment (start 63.075 75.075) (end 60.15 78) (width 0.25) (layer F.Cu) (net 2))
 (segment (start 59.5 71.9625) (end 56.5 71.9625) (width 0.25) (layer F.Cu) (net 2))
 (segment (start 58.45 77.05) (end 59.3 77.05) (width 0.25) (layer F.Cu) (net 4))
 (segment (start 58.374999 77.125001) (end 58.45 77.05) (width 0.25) (layer F.Cu) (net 4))
 (segment (start 58.374999 78.874999) (end 58.374999 77.125001) (width 0.25) (layer F.Cu) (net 4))
 (segment (start 58.45 78.95) (end 58.374999 78.874999) (width 0.25) (layer F.Cu) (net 4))
 (segment (start 59.3 78.95) (end 58.45 78.95) (width 0.25) (layer F.Cu) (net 4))
 (segment (start 64.6 78.95) (end 59.3 78.95) (width 0.25) (layer F.Cu) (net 4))
 (segment (start 65.7 77.85) (end 64.6 78.95) (width 0.25) (layer F.Cu) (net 4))
 (segment (start 59.3 74.2375) (end 59.5 74.0375) (width 0.25) (layer F.Cu) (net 4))
 (segment (start 59.3 77.05) (end 59.3 74.2375) (width 0.25) (layer F.Cu) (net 4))
 (segment (start 62.0375 71.5) (end 62.9 71.5) (width 0.25) (layer F.Cu) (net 6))
 (segment (start 60.0375 69.5) (end 62.0375 71.5) (width 0.25) (layer F.Cu) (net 6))
 (segment (start 62.564998 61.5) (end 62.9 61.5) (width 0.25) (layer F.Cu) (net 6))
 (segment (start 60.0375 64.027498) (end 62.564998 61.5) (width 0.25) (layer F.Cu) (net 6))
 (segment (start 71.5 47.5) (end 74 47.5) (width 0.25) (layer F.Cu) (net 6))
 (segment (start 71.5 45.54) (end 69.96 44) (width 0.25) (layer F.Cu) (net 6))
 (segment (start 71.5 47.5) (end 71.5 45.54) (width 0.25) (layer F.Cu) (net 6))
 (segment (start 63.235002 61.5) (end 62.9 61.5) (width 0.25) (layer F.Cu) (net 6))
 (segment (start 71.5 53.235002) (end 63.235002 61.5) (width 0.25) (layer F.Cu) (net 6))
 (segment (start 71.5 47.5) (end 71.5 53.235002) (width 0.25) (layer F.Cu) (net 6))
 (segment (start 55.774999 78.024999) (end 56.7 78.95) (width 0.25) (layer F.Cu) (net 6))
 (segment (start 55.774999 74.762501) (end 55.774999 78.024999) (width 0.25) (layer F.Cu) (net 6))
 (segment (start 56.5 74.0375) (end 55.774999 74.762501) (width 0.25) (layer F.Cu) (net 6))
 (segment (start 55.44999 71.38682) (end 58.79931 68.0375) (width 0.25) (layer F.Cu) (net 6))
 (segment (start 55.44999 72.98749) (end 55.44999 71.38682) (width 0.25) (layer F.Cu) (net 6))
 (segment (start 58.79931 68.0375) (end 60.0375 68.0375) (width 0.25) (layer F.Cu) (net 6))
 (segment (start 56.5 74.0375) (end 55.44999 72.98749) (width 0.25) (layer F.Cu) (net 6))
 (segment (start 60.0375 68.0375) (end 60.0375 64.027498) (width 0.25) (layer F.Cu) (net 6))
 (segment (start 60.0375 69.5) (end 60.0375 68.0375) (width 0.25) (layer F.Cu) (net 6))
 (segment (start 71.135001 40.284999) (end 69.96 41.46) (width 0.25) (layer F.Cu) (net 22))
 (segment (start 79.675001 44.355999) (end 75.604001 40.284999) (width 0.25) (layer F.Cu) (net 22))
 (segment (start 79.675001 61.424999) (end 79.675001 44.355999) (width 0.25) (layer F.Cu) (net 22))
 (segment (start 79.6 61.5) (end 79.675001 61.424999) (width 0.25) (layer F.Cu) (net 22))
 (segment (start 75.604001 40.284999) (end 71.135001 40.284999) (width 0.25) (layer F.Cu) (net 22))
 (segment (start 78.1 61.5) (end 79.6 61.5) (width 0.25) (layer F.Cu) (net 22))
 (segment (start 65.23 46.909998) (end 65.23 47.5) (width 0.25) (layer F.Cu) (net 3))
 (segment (start 75 44.04) (end 75.04 44) (width 0.25) (layer F.Cu) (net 3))
 (segment (start 65.15499 48.57501) (end 65.23 48.5) (width 0.25) (layer B.Cu) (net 3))
 (segment (start 63.10999 48.077085) (end 63.607915 48.57501) (width 0.25) (layer B.Cu) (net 3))
 (segment (start 69.395999 40.284999) (end 63.10999 46.571008) (width 0.25) (layer B.Cu) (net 3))
 (segment (start 75.604001 40.284999) (end 69.395999 40.284999) (width 0.25) (layer B.Cu) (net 3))
 (segment (start 63.607915 48.57501) (end 65.15499 48.57501) (width 0.25) (layer B.Cu) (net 3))
 (segment (start 76.215001 42.595997) (end 76.215001 40.895999) (width 0.25) (layer B.Cu) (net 3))
 (segment (start 76.215001 40.895999) (end 75.604001 40.284999) (width 0.25) (layer B.Cu) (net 3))
 (segment (start 75.889999 42.920999) (end 76.215001 42.595997) (width 0.25) (layer B.Cu) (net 3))
 (segment (start 65.23 48.5) (end 65.23 47.5) (width 0.25) (layer B.Cu) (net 3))
 (segment (start 63.10999 46.571008) (end 63.10999 48.077085) (width 0.25) (layer B.Cu) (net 3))
 (segment (start 75.889999 43.150001) (end 75.889999 42.920999) (width 0.25) (layer B.Cu) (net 3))
 (segment (start 75.04 44) (end 75.889999 43.150001) (width 0.25) (layer B.Cu) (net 3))
 (segment (start 76 44.96) (end 75.04 44) (width 0.25) (layer F.Cu) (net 3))
 (segment (start 76 47.5) (end 76 44.96) (width 0.25) (layer F.Cu) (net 3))
 (segment (start 69.96 47.46) (end 70 47.5) (width 0.25) (layer F.Cu) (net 1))
 (segment (start 69.5 47.5) (end 66.5 47.5) (width 0.25) (layer F.Cu) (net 1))
 (segment (start 66.5 45.174998) (end 66.5 47.5) (width 0.25) (layer F.Cu) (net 1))
 (segment (start 68.849999 42.824999) (end 66.5 45.174998) (width 0.25) (layer F.Cu) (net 1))
 (segment (start 71.135001 42.889999) (end 71.070001 42.824999) (width 0.25) (layer F.Cu) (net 1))
 (segment (start 71.135001 44.374003) (end 71.135001 42.889999) (width 0.25) (layer F.Cu) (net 1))
 (segment (start 71.935999 45.175001) (end 71.135001 44.374003) (width 0.25) (layer F.Cu) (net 1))
 (segment (start 73.288191 45.175001) (end 71.935999 45.175001) (width 0.25) (layer F.Cu) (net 1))
 (segment (start 74.92501 57.82501) (end 74.92501 46.81182) (width 0.25) (layer F.Cu) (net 1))
 (segment (start 71.070001 42.824999) (end 68.849999 42.824999) (width 0.25) (layer F.Cu) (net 1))
 (segment (start 74.92501 46.81182) (end 73.288191 45.175001) (width 0.25) (layer F.Cu) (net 1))
 (segment (start 76.6 59.5) (end 74.92501 57.82501) (width 0.25) (layer F.Cu) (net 1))
 (segment (start 78.1 59.5) (end 76.6 59.5) (width 0.25) (layer F.Cu) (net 1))
 (segment (start 78.6 70) (end 78.1 69.5) (width 0.25) (layer F.Cu) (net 5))
 (segment (start 81 70) (end 78.6 70) (width 0.25) (layer F.Cu) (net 5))
 (segment (start 64.475001 69.575001) (end 64.4 69.5) (width 0.25) (layer F.Cu) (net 12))
 (segment (start 64.4 69.5) (end 62.9 69.5) (width 0.25) (layer F.Cu) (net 12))
 (segment (start 74.914213 76) (end 80 76) (width 0.25) (layer F.Cu) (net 12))
 (segment (start 73.5 76) (end 74.914213 76) (width 0.25) (layer F.Cu) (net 12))
 (segment (start 65.985002 69.5) (end 62.9 69.5) (width 0.25) (layer F.Cu) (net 12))
 (segment (start 68.325001 71.839999) (end 65.985002 69.5) (width 0.25) (layer F.Cu) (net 12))
 (segment (start 68.325001 73.810003) (end 68.325001 71.839999) (width 0.25) (layer F.Cu) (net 12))
 (segment (start 70.514998 76) (end 68.325001 73.810003) (width 0.25) (layer F.Cu) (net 12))
 (segment (start 73.5 76) (end 70.514998 76) (width 0.25) (layer F.Cu) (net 12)))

